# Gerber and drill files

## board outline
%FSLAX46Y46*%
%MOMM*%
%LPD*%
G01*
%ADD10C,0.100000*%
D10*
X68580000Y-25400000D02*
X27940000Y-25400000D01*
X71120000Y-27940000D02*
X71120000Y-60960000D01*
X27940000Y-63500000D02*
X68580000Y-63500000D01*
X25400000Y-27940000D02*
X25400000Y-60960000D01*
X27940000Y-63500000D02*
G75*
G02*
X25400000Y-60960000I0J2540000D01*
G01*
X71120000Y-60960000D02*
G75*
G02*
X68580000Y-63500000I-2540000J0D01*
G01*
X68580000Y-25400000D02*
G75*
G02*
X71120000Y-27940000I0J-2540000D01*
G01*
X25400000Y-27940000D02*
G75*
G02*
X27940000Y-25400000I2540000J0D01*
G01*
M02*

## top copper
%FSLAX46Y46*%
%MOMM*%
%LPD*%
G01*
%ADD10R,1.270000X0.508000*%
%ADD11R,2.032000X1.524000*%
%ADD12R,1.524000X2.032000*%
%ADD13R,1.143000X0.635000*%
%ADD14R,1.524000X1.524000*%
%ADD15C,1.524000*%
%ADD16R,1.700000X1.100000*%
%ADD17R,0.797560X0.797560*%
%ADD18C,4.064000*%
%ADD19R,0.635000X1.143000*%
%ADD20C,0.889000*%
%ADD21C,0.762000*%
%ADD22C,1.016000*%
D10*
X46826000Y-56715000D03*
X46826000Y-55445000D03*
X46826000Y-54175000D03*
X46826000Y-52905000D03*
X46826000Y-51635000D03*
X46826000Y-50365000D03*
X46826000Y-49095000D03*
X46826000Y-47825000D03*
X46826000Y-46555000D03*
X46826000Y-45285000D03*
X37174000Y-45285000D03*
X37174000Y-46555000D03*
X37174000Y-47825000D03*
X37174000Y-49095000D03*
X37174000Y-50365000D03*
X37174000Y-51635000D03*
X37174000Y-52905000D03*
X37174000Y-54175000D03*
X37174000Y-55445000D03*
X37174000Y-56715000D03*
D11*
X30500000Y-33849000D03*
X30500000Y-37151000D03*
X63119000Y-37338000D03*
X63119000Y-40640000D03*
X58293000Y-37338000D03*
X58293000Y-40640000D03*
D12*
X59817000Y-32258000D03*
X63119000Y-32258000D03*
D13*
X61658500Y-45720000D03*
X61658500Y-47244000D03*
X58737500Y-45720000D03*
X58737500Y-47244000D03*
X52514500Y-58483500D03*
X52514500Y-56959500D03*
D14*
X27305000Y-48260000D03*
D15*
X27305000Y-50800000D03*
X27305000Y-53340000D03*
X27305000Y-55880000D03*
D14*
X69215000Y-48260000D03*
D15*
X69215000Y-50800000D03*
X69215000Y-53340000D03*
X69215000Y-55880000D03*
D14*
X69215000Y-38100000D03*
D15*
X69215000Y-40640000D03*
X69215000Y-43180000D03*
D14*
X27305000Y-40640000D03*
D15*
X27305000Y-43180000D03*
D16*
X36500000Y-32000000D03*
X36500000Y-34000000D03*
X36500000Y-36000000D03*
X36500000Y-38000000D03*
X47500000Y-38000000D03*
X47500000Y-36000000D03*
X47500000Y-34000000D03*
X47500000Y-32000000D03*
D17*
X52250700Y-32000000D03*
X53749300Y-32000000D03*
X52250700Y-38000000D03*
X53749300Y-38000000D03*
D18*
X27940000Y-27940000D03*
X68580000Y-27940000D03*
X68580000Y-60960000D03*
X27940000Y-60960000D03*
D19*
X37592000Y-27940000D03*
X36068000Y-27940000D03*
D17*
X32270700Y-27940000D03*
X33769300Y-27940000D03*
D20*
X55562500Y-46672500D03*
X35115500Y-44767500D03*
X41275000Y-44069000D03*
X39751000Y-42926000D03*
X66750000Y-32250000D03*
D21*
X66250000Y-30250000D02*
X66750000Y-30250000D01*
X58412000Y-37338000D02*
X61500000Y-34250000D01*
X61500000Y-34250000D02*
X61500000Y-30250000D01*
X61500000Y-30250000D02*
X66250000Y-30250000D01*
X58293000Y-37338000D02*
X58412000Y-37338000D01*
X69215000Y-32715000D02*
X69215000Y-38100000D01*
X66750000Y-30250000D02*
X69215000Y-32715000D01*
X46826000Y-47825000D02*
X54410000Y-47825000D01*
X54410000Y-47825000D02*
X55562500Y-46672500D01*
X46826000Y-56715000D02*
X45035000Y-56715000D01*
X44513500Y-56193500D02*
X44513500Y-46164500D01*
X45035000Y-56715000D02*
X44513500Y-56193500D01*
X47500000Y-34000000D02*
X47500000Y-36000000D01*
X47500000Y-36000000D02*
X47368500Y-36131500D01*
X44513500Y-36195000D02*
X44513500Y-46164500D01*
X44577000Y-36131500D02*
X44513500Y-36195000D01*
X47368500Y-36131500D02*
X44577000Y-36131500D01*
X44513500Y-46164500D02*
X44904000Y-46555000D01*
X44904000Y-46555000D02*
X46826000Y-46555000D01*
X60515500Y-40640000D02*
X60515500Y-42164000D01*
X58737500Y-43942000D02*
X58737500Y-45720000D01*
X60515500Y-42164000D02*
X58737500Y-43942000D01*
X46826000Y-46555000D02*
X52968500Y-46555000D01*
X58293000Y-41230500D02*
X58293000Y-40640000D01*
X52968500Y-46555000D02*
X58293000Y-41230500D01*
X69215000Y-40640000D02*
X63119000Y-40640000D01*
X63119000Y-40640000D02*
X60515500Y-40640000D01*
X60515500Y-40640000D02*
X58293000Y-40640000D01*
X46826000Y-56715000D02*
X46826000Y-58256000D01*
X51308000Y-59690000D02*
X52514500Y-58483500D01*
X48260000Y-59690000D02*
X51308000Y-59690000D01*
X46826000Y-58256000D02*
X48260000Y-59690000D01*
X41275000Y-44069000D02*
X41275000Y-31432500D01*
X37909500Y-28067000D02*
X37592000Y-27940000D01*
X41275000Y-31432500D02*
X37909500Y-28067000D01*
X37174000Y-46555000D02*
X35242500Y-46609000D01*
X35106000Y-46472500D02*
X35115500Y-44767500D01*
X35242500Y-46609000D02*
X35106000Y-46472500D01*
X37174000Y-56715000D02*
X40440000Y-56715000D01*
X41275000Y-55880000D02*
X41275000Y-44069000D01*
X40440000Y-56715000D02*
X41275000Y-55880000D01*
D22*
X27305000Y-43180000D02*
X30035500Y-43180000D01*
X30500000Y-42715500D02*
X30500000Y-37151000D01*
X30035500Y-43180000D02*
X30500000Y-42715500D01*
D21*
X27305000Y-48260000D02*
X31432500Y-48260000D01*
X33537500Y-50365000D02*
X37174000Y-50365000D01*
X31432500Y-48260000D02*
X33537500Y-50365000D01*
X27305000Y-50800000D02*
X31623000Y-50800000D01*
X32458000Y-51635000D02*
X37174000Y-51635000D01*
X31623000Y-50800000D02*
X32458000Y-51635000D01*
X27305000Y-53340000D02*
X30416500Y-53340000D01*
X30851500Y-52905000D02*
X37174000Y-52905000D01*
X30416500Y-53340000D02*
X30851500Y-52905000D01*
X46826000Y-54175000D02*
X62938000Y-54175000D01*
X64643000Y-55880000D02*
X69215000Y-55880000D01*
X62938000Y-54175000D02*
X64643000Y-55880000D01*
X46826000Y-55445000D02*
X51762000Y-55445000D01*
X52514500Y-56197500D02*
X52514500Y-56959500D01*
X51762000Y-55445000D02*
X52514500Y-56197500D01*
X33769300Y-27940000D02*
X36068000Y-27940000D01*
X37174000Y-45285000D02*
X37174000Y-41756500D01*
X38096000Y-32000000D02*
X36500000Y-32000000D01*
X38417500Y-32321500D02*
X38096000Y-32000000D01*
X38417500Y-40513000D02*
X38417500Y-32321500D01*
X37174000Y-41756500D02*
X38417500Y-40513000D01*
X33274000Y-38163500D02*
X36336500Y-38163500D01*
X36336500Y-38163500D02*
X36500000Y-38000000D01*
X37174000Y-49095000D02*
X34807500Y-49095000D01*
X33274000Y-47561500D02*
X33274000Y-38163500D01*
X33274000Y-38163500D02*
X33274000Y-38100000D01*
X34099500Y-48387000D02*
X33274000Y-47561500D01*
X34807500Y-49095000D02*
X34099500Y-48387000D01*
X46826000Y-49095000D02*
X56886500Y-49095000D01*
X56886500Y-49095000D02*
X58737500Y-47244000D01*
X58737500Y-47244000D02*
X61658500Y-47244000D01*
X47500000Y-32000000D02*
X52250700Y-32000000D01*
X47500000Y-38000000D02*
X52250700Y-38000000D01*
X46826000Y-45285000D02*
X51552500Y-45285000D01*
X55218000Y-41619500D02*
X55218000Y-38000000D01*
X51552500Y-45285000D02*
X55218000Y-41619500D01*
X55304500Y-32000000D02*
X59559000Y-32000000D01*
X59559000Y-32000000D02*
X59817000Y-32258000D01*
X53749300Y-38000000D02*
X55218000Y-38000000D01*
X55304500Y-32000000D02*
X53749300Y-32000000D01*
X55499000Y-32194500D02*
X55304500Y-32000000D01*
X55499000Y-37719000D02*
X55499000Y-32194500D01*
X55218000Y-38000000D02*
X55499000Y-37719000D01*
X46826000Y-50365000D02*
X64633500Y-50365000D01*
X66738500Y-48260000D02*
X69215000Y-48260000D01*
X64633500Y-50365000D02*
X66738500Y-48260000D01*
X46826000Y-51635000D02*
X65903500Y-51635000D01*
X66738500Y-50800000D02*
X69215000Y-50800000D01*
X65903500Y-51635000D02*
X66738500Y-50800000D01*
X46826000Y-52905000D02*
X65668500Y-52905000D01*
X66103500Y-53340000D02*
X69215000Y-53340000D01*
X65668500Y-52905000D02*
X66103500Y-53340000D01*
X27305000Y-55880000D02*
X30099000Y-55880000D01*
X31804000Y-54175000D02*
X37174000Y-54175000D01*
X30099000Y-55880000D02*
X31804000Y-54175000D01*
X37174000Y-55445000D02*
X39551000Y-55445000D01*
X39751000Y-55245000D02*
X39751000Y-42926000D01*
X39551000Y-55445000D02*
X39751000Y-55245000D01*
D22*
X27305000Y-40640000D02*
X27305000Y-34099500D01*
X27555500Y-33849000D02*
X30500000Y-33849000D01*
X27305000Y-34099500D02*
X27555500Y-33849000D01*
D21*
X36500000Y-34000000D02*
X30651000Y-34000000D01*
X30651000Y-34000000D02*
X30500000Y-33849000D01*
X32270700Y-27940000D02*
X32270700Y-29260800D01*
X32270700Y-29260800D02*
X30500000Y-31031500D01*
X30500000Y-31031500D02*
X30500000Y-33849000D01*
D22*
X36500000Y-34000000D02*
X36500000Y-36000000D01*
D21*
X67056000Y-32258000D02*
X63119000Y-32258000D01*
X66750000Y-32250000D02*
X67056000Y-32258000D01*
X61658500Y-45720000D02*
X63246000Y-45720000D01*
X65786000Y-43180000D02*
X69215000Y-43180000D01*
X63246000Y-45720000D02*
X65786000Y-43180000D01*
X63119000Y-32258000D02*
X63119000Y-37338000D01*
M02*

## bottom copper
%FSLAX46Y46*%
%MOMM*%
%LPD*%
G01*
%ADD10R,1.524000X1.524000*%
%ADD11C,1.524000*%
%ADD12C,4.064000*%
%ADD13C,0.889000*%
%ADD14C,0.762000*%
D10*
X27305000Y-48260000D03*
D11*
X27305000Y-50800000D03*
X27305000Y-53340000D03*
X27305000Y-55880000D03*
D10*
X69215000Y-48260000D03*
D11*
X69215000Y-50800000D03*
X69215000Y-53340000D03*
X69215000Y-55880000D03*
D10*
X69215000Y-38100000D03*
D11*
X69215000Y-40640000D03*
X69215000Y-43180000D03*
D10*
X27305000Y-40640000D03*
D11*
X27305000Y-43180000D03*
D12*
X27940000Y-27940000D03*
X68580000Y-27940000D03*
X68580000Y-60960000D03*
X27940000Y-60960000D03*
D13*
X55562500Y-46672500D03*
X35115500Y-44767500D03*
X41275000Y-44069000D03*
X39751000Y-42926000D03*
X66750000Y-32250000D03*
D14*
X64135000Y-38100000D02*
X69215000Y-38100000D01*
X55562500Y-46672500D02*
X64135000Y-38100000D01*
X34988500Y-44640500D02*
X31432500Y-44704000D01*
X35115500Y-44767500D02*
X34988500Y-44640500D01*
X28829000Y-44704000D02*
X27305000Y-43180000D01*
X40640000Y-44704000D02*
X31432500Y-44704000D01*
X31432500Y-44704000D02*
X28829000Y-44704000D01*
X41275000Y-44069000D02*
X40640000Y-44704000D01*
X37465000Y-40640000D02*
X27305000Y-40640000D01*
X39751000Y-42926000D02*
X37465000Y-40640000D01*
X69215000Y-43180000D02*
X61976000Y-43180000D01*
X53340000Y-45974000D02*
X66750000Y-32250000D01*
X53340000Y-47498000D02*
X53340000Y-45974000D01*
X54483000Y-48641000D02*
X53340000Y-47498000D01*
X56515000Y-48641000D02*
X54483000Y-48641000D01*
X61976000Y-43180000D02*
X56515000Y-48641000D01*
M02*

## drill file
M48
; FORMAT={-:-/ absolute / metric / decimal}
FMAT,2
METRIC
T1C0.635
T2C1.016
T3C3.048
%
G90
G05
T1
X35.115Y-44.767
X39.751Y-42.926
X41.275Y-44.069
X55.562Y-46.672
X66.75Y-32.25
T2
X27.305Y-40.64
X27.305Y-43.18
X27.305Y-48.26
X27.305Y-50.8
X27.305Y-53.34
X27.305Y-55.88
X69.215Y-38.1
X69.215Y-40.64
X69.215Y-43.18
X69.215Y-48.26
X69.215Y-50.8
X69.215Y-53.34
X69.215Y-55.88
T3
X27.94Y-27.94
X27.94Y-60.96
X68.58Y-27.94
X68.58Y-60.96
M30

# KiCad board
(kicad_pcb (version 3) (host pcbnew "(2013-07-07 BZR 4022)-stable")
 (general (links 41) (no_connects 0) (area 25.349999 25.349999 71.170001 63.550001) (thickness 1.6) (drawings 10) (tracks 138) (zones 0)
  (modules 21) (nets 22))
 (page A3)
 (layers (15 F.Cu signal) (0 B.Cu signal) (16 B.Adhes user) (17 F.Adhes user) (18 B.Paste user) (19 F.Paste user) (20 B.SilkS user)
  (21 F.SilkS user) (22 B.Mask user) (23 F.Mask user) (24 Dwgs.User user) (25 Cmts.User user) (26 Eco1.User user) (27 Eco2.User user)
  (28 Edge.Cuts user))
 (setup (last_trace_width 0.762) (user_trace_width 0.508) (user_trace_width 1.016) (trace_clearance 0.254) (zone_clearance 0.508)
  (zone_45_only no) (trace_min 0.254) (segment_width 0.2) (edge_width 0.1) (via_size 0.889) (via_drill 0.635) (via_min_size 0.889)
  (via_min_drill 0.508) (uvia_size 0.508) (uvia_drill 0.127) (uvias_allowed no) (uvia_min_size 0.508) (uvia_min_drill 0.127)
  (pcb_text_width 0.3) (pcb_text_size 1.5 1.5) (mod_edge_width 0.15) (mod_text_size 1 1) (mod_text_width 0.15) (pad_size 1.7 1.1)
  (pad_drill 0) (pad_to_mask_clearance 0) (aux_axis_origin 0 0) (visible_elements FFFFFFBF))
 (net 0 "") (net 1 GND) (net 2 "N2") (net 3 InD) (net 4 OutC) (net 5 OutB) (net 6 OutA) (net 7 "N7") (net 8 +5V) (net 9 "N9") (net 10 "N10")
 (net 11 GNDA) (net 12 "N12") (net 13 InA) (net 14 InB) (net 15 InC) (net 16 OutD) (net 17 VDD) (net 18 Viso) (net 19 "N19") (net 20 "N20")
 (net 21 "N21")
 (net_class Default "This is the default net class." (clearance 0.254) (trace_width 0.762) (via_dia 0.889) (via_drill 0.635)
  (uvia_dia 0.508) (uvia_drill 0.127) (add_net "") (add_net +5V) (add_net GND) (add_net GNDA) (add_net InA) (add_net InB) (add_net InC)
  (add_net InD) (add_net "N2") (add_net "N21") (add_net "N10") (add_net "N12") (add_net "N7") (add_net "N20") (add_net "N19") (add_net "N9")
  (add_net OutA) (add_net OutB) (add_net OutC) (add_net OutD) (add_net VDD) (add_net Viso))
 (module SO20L (layer F.Cu) (at 42 51 270)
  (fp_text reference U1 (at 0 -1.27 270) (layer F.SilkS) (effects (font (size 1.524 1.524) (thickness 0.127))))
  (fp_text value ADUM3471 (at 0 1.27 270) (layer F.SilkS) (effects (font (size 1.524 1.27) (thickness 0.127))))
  (pad 11 smd rect (at 5.715 -4.826 270) (size 0.508 1.27) (layers F.Cu F.Paste F.Mask) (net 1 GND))
  (pad 12 smd rect (at 4.445 -4.826 270) (size 0.508 1.27) (layers F.Cu F.Paste F.Mask) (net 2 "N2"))
  (pad 13 smd rect (at 3.175 -4.826 270) (size 0.508 1.27) (layers F.Cu F.Paste F.Mask) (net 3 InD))
  (pad 14 smd rect (at 1.905 -4.826 270) (size 0.508 1.27) (layers F.Cu F.Paste F.Mask) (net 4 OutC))
  (pad 15 smd rect (at 0.635 -4.826 270) (size 0.508 1.27) (layers F.Cu F.Paste F.Mask) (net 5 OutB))
  (pad 16 smd rect (at -0.635 -4.826 270) (size 0.508 1.27) (layers F.Cu F.Paste F.Mask) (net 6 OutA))
  (pad 17 smd rect (at -1.905 -4.826 270) (size 0.508 1.27) (layers F.Cu F.Paste F.Mask) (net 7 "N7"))
  (pad 18 smd rect (at -3.175 -4.826 270) (size 0.508 1.27) (layers F.Cu F.Paste F.Mask) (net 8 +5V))
  (pad 19 smd rect (at -4.445 -4.826 270) (size 0.508 1.27) (layers F.Cu F.Paste F.Mask) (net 1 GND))
  (pad 20 smd rect (at -5.715 -4.826 270) (size 0.508 1.27) (layers F.Cu F.Paste F.Mask) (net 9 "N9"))
  (pad 1 smd rect (at -5.715 4.826 270) (size 0.508 1.27) (layers F.Cu F.Paste F.Mask) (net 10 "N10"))
  (pad 2 smd rect (at -4.445 4.826 270) (size 0.508 1.27) (layers F.Cu F.Paste F.Mask) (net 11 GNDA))
  (pad 3 smd rect (at -3.175 4.826 270) (size 0.508 1.27) (layers F.Cu F.Paste F.Mask))
  (pad 4 smd rect (at -1.905 4.826 270) (size 0.508 1.27) (layers F.Cu F.Paste F.Mask) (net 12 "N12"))
  (pad 5 smd rect (at -0.635 4.826 270) (size 0.508 1.27) (layers F.Cu F.Paste F.Mask) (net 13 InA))
  (pad 6 smd rect (at 0.635 4.826 270) (size 0.508 1.27) (layers F.Cu F.Paste F.Mask) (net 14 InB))
  (pad 7 smd rect (at 1.905 4.826 270) (size 0.508 1.27) (layers F.Cu F.Paste F.Mask) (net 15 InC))
  (pad 8 smd rect (at 3.175 4.826 270) (size 0.508 1.27) (layers F.Cu F.Paste F.Mask) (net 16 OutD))
  (pad 9 smd rect (at 4.445 4.826 270) (size 0.508 1.27) (layers F.Cu F.Paste F.Mask) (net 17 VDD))
  (pad 10 smd rect (at 5.715 4.826 270) (size 0.508 1.27) (layers F.Cu F.Paste F.Mask) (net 11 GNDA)))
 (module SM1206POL (layer F.Cu) (at 30.5 35.5 270)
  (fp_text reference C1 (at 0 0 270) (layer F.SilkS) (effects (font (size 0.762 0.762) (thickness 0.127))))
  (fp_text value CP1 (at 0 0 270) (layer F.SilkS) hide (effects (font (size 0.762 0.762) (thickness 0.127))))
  (pad 1 smd rect (at -1.651 0 270) (size 1.524 2.032) (layers F.Cu F.Paste F.Mask) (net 17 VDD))
  (pad 2 smd rect (at 1.651 0 270) (size 1.524 2.032) (layers F.Cu F.Paste F.Mask) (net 11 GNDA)))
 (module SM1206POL (layer F.Cu) (at 63.119 38.989 270)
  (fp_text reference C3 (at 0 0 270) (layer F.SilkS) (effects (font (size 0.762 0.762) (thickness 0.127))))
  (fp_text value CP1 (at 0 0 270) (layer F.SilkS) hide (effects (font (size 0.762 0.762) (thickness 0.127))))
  (pad 1 smd rect (at -1.651 0 270) (size 1.524 2.032) (layers F.Cu F.Paste F.Mask) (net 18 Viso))
  (pad 2 smd rect (at 1.651 0 270) (size 1.524 2.032) (layers F.Cu F.Paste F.Mask) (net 1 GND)))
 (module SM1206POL (layer F.Cu) (at 58.293 38.989 270)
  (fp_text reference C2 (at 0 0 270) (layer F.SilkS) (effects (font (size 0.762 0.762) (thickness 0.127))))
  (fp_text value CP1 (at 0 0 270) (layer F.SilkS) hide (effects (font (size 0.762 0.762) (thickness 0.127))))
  (pad 1 smd rect (at -1.651 0 270) (size 1.524 2.032) (layers F.Cu F.Paste F.Mask) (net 8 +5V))
  (pad 2 smd rect (at 1.651 0 270) (size 1.524 2.032) (layers F.Cu F.Paste F.Mask) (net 1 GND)))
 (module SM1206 (layer F.Cu) (at 61.468 32.258)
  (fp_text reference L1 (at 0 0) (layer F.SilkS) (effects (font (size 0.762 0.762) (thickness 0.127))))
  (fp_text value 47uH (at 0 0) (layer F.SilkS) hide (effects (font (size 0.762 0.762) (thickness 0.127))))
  (pad 1 smd rect (at -1.651 0) (size 1.524 2.032) (layers F.Cu F.Paste F.Mask) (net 9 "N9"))
  (pad 2 smd rect (at 1.651 0) (size 1.524 2.032) (layers F.Cu F.Paste F.Mask) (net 18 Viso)))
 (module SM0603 (layer F.Cu) (at 61.6585 46.482 270)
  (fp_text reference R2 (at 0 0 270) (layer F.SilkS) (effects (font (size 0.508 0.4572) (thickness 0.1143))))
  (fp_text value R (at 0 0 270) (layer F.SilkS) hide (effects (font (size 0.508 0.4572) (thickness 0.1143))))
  (pad 1 smd rect (at -0.762 0 270) (size 0.635 1.143) (layers F.Cu F.Paste F.Mask) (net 18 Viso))
  (pad 2 smd rect (at 0.762 0 270) (size 0.635 1.143) (layers F.Cu F.Paste F.Mask) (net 7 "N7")))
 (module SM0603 (layer F.Cu) (at 58.7375 46.482 270)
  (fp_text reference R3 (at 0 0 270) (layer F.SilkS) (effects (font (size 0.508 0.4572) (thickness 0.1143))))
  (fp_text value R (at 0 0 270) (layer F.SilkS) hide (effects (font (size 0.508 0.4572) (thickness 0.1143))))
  (pad 1 smd rect (at -0.762 0 270) (size 0.635 1.143) (layers F.Cu F.Paste F.Mask) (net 1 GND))
  (pad 2 smd rect (at 0.762 0 270) (size 0.635 1.143) (layers F.Cu F.Paste F.Mask) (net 7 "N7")))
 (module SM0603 (layer F.Cu) (at 52.5145 57.7215 90)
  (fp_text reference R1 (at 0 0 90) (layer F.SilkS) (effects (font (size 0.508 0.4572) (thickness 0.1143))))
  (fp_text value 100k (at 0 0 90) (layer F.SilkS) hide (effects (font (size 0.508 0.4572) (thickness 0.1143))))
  (pad 1 smd rect (at -0.762 0 90) (size 0.635 1.143) (layers F.Cu F.Paste F.Mask) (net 1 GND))
  (pad 2 smd rect (at 0.762 0 90) (size 0.635 1.143) (layers F.Cu F.Paste F.Mask) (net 2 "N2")))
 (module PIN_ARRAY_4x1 (layer F.Cu) (at 27.305 52.07 270)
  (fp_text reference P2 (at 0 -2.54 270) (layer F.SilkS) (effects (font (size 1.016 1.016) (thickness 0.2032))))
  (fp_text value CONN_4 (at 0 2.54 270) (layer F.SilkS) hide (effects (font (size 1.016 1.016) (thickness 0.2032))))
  (pad 1 thru_hole rect (at -3.81 0 270) (size 1.524 1.524) (drill 1.016) (layers *.Cu *.Mask F.SilkS) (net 13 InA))
  (pad 2 thru_hole circle (at -1.27 0 270) (size 1.524 1.524) (drill 1.016) (layers *.Cu *.Mask F.SilkS) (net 14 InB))
  (pad 3 thru_hole circle (at 1.27 0 270) (size 1.524 1.524) (drill 1.016) (layers *.Cu *.Mask F.SilkS) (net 15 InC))
  (pad 4 thru_hole circle (at 3.81 0 270) (size 1.524 1.524) (drill 1.016) (layers *.Cu *.Mask F.SilkS) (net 16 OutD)))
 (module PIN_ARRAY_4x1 (layer F.Cu) (at 69.215 52.07 270)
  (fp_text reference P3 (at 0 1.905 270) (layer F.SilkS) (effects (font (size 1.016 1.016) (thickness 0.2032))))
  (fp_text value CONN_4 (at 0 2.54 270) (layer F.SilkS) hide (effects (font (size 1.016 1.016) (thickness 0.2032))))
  (pad 1 thru_hole rect (at -3.81 0 270) (size 1.524 1.524) (drill 1.016) (layers *.Cu *.Mask F.SilkS) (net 6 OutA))
  (pad 2 thru_hole circle (at -1.27 0 270) (size 1.524 1.524) (drill 1.016) (layers *.Cu *.Mask F.SilkS) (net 5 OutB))
  (pad 3 thru_hole circle (at 1.27 0 270) (size 1.524 1.524) (drill 1.016) (layers *.Cu *.Mask F.SilkS) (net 4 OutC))
  (pad 4 thru_hole circle (at 3.81 0 270) (size 1.524 1.524) (drill 1.016) (layers *.Cu *.Mask F.SilkS) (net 3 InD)))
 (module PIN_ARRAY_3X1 (layer F.Cu) (at 69.215 40.64 270)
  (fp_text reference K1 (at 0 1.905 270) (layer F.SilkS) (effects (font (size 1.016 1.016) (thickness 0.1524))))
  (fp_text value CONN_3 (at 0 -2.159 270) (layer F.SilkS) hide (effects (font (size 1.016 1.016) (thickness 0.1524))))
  (pad 1 thru_hole rect (at -2.54 0 270) (size 1.524 1.524) (drill 1.016) (layers *.Cu *.Mask F.SilkS) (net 8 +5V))
  (pad 2 thru_hole circle (at 0 0 270) (size 1.524 1.524) (drill 1.016) (layers *.Cu *.Mask F.SilkS) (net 1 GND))
  (pad 3 thru_hole circle (at 2.54 0 270) (size 1.524 1.524) (drill 1.016) (layers *.Cu *.Mask F.SilkS) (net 18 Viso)))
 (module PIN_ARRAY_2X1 (layer F.Cu) (at 27.305 41.91 270)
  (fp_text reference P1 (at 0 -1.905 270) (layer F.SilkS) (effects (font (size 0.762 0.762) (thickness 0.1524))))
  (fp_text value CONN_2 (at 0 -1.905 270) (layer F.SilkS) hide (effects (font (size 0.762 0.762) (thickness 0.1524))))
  (pad 1 thru_hole rect (at -1.27 0 270) (size 1.524 1.524) (drill 1.016) (layers *.Cu *.Mask F.SilkS) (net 17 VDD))
  (pad 2 thru_hole circle (at 1.27 0 270) (size 1.524 1.524) (drill 1.016) (layers *.Cu *.Mask F.SilkS) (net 11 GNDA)))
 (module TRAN (layer F.Cu) (at 42 35)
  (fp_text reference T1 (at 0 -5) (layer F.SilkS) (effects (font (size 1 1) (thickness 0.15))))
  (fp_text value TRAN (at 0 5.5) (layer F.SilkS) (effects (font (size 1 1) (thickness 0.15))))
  (pad 1 smd rect (at -5.5 -3) (size 1.7 1.1) (layers F.Cu F.Paste F.Mask) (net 10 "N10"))
  (pad 2 smd rect (at -5.5 -1) (size 1.7 1.1) (layers F.Cu F.Paste F.Mask) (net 17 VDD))
  (pad 3 smd rect (at -5.5 1) (size 1.7 1.1) (layers F.Cu F.Paste F.Mask) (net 17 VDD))
  (pad 4 smd rect (at -5.5 3) (size 1.7 1.1) (layers F.Cu F.Paste F.Mask) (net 12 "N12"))
  (pad 5 smd rect (at 5.5 3) (size 1.7 1.1) (layers F.Cu F.Paste F.Mask) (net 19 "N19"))
  (pad 6 smd rect (at 5.5 1) (size 1.7 1.1) (layers F.Cu F.Paste F.Mask) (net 1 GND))
  (pad 7 smd rect (at 5.5 -1) (size 1.7 1.1) (layers F.Cu F.Paste F.Mask) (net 1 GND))
  (pad 8 smd rect (at 5.5 -3) (size 1.7 1.1) (layers F.Cu F.Paste F.Mask) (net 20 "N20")))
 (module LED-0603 (layer F.Cu) (at 53 32)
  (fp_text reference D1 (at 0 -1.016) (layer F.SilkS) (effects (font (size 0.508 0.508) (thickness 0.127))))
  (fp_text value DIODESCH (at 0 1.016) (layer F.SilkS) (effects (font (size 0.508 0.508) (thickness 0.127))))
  (pad 1 smd rect (at -0.7493 0) (size 0.79756 0.79756) (layers F.Cu F.Paste F.Mask) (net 20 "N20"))
  (pad 2 smd rect (at 0.7493 0) (size 0.79756 0.79756) (layers F.Cu F.Paste F.Mask) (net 9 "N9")))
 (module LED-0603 (layer F.Cu) (at 53 38)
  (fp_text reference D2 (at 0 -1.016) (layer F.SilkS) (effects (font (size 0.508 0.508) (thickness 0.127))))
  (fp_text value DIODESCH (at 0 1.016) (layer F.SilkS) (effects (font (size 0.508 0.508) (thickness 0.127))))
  (pad 1 smd rect (at -0.7493 0) (size 0.79756 0.79756) (layers F.Cu F.Paste F.Mask) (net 19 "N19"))
  (pad 2 smd rect (at 0.7493 0) (size 0.79756 0.79756) (layers F.Cu F.Paste F.Mask) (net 9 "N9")))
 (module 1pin (layer F.Cu) (at 27.94 27.94)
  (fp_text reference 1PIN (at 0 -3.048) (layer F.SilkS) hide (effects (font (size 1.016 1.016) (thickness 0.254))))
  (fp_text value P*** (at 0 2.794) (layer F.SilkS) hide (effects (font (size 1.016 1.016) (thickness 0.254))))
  (pad 1 thru_hole circle (at 0 0) (size 4.064 4.064) (drill 3.048) (layers *.Cu *.Mask F.SilkS)))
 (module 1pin (layer F.Cu) (at 68.58 27.94)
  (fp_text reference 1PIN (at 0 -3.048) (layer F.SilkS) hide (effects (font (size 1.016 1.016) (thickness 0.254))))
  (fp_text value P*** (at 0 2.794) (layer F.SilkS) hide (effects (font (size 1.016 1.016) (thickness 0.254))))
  (pad 1 thru_hole circle (at 0 0) (size 4.064 4.064) (drill 3.048) (layers *.Cu *.Mask F.SilkS)))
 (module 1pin (layer F.Cu) (at 68.58 60.96)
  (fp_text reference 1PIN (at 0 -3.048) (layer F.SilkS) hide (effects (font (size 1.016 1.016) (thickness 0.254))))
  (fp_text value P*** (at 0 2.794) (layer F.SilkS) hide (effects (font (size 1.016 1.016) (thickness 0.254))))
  (pad 1 thru_hole circle (at 0 0) (size 4.064 4.064) (drill 3.048) (layers *.Cu *.Mask F.SilkS)))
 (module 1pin (layer F.Cu) (at 27.94 60.96)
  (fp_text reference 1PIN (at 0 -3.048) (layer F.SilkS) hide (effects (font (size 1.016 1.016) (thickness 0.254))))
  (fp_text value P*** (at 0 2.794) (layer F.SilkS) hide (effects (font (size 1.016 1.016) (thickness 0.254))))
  (pad 1 thru_hole circle (at 0 0) (size 4.064 4.064) (drill 3.048) (layers *.Cu *.Mask F.SilkS)))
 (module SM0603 (layer F.Cu) (at 36.83 27.94 180)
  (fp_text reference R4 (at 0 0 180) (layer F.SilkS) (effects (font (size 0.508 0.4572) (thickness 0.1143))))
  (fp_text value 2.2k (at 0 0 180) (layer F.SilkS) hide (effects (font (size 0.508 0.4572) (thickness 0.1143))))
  (pad 1 smd rect (at -0.762 0 180) (size 0.635 1.143) (layers F.Cu F.Paste F.Mask) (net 11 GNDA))
  (pad 2 smd rect (at 0.762 0 180) (size 0.635 1.143) (layers F.Cu F.Paste F.Mask) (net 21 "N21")))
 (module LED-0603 (layer F.Cu) (at 33.02 27.94)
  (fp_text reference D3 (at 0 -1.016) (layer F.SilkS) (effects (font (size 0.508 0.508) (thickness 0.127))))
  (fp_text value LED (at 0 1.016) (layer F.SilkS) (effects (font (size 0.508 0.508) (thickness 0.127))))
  (pad 1 smd rect (at -0.7493 0) (size 0.79756 0.79756) (layers F.Cu F.Paste F.Mask) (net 17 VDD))
  (pad 2 smd rect (at 0.7493 0) (size 0.79756 0.79756) (layers F.Cu F.Paste F.Mask) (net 21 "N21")))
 (gr_line (start 68.58 25.4) (end 27.94 25.4) (angle 90) (layer Edge.Cuts) (width 0.1))
 (gr_line (start 71.12 27.94) (end 71.12 60.96) (angle 90) (layer Edge.Cuts) (width 0.1))
 (gr_line (start 27.94 63.5) (end 68.58 63.5) (angle 90) (layer Edge.Cuts) (width 0.1))
 (gr_line (start 25.4 27.94) (end 25.4 60.96) (angle 90) (layer Edge.Cuts) (width 0.1))
 (gr_arc (start 27.94 60.96) (end 27.94 63.5) (angle 90) (layer Edge.Cuts) (width 0.1))
 (gr_arc (start 68.58 60.96) (end 71.12 60.96) (angle 90) (layer Edge.Cuts) (width 0.1))
 (gr_arc (start 68.58 27.94) (end 68.58 25.4) (angle 90) (layer Edge.Cuts) (width 0.1))
 (gr_arc (start 27.94 27.94) (end 25.4 27.94) (angle 90) (layer Edge.Cuts) (width 0.1))
 (segment (start 66.25 30.25) (end 66.75 30.25) (width 0.762) (layer F.Cu) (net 8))
 (segment (start 58.412 37.338) (end 61.5 34.25) (width 0.762) (layer F.Cu) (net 8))
 (segment (start 61.5 34.25) (end 61.5 30.25) (width 0.762) (layer F.Cu) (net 8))
 (segment (start 61.5 30.25) (end 66.25 30.25) (width 0.762) (layer F.Cu) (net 8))
 (segment (start 58.293 37.338) (end 58.412 37.338) (width 0.762) (layer F.Cu) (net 8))
 (segment (start 69.215 32.715) (end 69.215 38.1) (width 0.762) (layer F.Cu) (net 8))
 (segment (start 66.75 30.25) (end 69.215 32.715) (width 0.762) (layer F.Cu) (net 8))
 (segment (start 46.826 47.825) (end 54.41 47.825) (width 0.762) (layer F.Cu) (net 8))
 (segment (start 64.135 38.1) (end 69.215 38.1) (width 0.762) (layer B.Cu) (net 8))
 (segment (start 55.5625 46.6725) (end 64.135 38.1) (width 0.762) (layer B.Cu) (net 8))
 (via (at 55.5625 46.6725) (size 0.889) (layers F.Cu B.Cu) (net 8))
 (segment (start 54.41 47.825) (end 55.5625 46.6725) (width 0.762) (layer F.Cu) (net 8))
 (segment (start 46.826 56.715) (end 45.035 56.715) (width 0.762) (layer F.Cu) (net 1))
 (segment (start 44.5135 56.1935) (end 44.5135 46.1645) (width 0.762) (layer F.Cu) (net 1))
 (segment (start 45.035 56.715) (end 44.5135 56.1935) (width 0.762) (layer F.Cu) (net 1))
 (segment (start 47.5 34) (end 47.5 36) (width 0.762) (layer F.Cu) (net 1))
 (segment (start 47.5 36) (end 47.3685 36.1315) (width 0.762) (layer F.Cu) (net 1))
 (segment (start 44.5135 36.195) (end 44.5135 46.1645) (width 0.762) (layer F.Cu) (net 1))
 (segment (start 44.577 36.1315) (end 44.5135 36.195) (width 0.762) (layer F.Cu) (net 1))
 (segment (start 47.3685 36.1315) (end 44.577 36.1315) (width 0.762) (layer F.Cu) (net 1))
 (segment (start 44.5135 46.1645) (end 44.904 46.555) (width 0.762) (layer F.Cu) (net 1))
 (segment (start 44.904 46.555) (end 46.826 46.555) (width 0.762) (layer F.Cu) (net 1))
 (segment (start 60.5155 40.64) (end 60.5155 42.164) (width 0.762) (layer F.Cu) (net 1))
 (segment (start 58.7375 43.942) (end 58.7375 45.72) (width 0.762) (layer F.Cu) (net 1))
 (segment (start 60.5155 42.164) (end 58.7375 43.942) (width 0.762) (layer F.Cu) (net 1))
 (segment (start 46.826 46.555) (end 52.9685 46.555) (width 0.762) (layer F.Cu) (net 1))
 (segment (start 58.293 41.2305) (end 58.293 40.64) (width 0.762) (layer F.Cu) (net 1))
 (segment (start 52.9685 46.555) (end 58.293 41.2305) (width 0.762) (layer F.Cu) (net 1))
 (segment (start 69.215 40.64) (end 63.119 40.64) (width 0.762) (layer F.Cu) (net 1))
 (segment (start 63.119 40.64) (end 60.5155 40.64) (width 0.762) (layer F.Cu) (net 1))
 (segment (start 60.5155 40.64) (end 58.293 40.64) (width 0.762) (layer F.Cu) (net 1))
 (segment (start 46.826 56.715) (end 46.826 58.256) (width 0.762) (layer F.Cu) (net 1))
 (segment (start 51.308 59.69) (end 52.5145 58.4835) (width 0.762) (layer F.Cu) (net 1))
 (segment (start 48.26 59.69) (end 51.308 59.69) (width 0.762) (layer F.Cu) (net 1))
 (segment (start 46.826 58.256) (end 48.26 59.69) (width 0.762) (layer F.Cu) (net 1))
 (segment (start 41.275 44.069) (end 41.275 31.4325) (width 0.762) (layer F.Cu) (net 11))
 (segment (start 37.9095 28.067) (end 37.592 27.94) (width 0.762) (layer F.Cu) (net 11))
 (segment (start 41.275 31.4325) (end 37.9095 28.067) (width 0.762) (layer F.Cu) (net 11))
 (segment (start 37.174 46.555) (end 35.2425 46.609) (width 0.762) (layer F.Cu) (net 11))
 (segment (start 34.9885 44.6405) (end 31.4325 44.704) (width 0.762) (layer B.Cu) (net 11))
 (segment (start 35.1155 44.7675) (end 34.9885 44.6405) (width 0.762) (layer B.Cu) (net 11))
 (via (at 35.1155 44.7675) (size 0.889) (layers F.Cu B.Cu) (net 11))
 (segment (start 35.106 46.4725) (end 35.1155 44.7675) (width 0.762) (layer F.Cu) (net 11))
 (segment (start 35.2425 46.609) (end 35.106 46.4725) (width 0.762) (layer F.Cu) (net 11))
 (segment (start 37.174 56.715) (end 40.44 56.715) (width 0.762) (layer F.Cu) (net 11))
 (segment (start 28.829 44.704) (end 27.305 43.18) (width 0.762) (layer B.Cu) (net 11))
 (segment (start 40.64 44.704) (end 31.4325 44.704) (width 0.762) (layer B.Cu) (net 11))
 (segment (start 31.4325 44.704) (end 28.829 44.704) (width 0.762) (layer B.Cu) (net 11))
 (segment (start 41.275 44.069) (end 40.64 44.704) (width 0.762) (layer B.Cu) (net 11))
 (via (at 41.275 44.069) (size 0.889) (layers F.Cu B.Cu) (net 11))
 (segment (start 41.275 55.88) (end 41.275 44.069) (width 0.762) (layer F.Cu) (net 11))
 (segment (start 40.44 56.715) (end 41.275 55.88) (width 0.762) (layer F.Cu) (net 11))
 (segment (start 27.305 43.18) (end 30.0355 43.18) (width 1.016) (layer F.Cu) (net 11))
 (segment (start 30.5 42.7155) (end 30.5 37.151) (width 1.016) (layer F.Cu) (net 11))
 (segment (start 30.0355 43.18) (end 30.5 42.7155) (width 1.016) (layer F.Cu) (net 11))
 (segment (start 27.305 48.26) (end 31.4325 48.26) (width 0.762) (layer F.Cu) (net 13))
 (segment (start 33.5375 50.365) (end 37.174 50.365) (width 0.762) (layer F.Cu) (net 13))
 (segment (start 31.4325 48.26) (end 33.5375 50.365) (width 0.762) (layer F.Cu) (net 13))
 (segment (start 27.305 50.8) (end 31.623 50.8) (width 0.762) (layer F.Cu) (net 14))
 (segment (start 32.458 51.635) (end 37.174 51.635) (width 0.762) (layer F.Cu) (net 14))
 (segment (start 31.623 50.8) (end 32.458 51.635) (width 0.762) (layer F.Cu) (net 14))
 (segment (start 27.305 53.34) (end 30.4165 53.34) (width 0.762) (layer F.Cu) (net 15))
 (segment (start 30.8515 52.905) (end 37.174 52.905) (width 0.762) (layer F.Cu) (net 15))
 (segment (start 30.4165 53.34) (end 30.8515 52.905) (width 0.762) (layer F.Cu) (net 15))
 (segment (start 46.826 54.175) (end 62.938 54.175) (width 0.762) (layer F.Cu) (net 3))
 (segment (start 64.643 55.88) (end 69.215 55.88) (width 0.762) (layer F.Cu) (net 3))
 (segment (start 62.938 54.175) (end 64.643 55.88) (width 0.762) (layer F.Cu) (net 3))
 (segment (start 46.826 55.445) (end 51.762 55.445) (width 0.762) (layer F.Cu) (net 2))
 (segment (start 52.5145 56.1975) (end 52.5145 56.9595) (width 0.762) (layer F.Cu) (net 2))
 (segment (start 51.762 55.445) (end 52.5145 56.1975) (width 0.762) (layer F.Cu) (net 2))
 (segment (start 33.7693 27.94) (end 36.068 27.94) (width 0.762) (layer F.Cu) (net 21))
 (segment (start 37.174 45.285) (end 37.174 41.7565) (width 0.762) (layer F.Cu) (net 10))
 (segment (start 38.096 32) (end 36.5 32) (width 0.762) (layer F.Cu) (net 10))
 (segment (start 38.4175 32.3215) (end 38.096 32) (width 0.762) (layer F.Cu) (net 10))
 (segment (start 38.4175 40.513) (end 38.4175 32.3215) (width 0.762) (layer F.Cu) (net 10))
 (segment (start 37.174 41.7565) (end 38.4175 40.513) (width 0.762) (layer F.Cu) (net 10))
 (segment (start 33.274 38.1635) (end 36.3365 38.1635) (width 0.762) (layer F.Cu) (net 12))
 (segment (start 36.3365 38.1635) (end 36.5 38) (width 0.762) (layer F.Cu) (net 12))
 (segment (start 37.174 49.095) (end 34.8075 49.095) (width 0.762) (layer F.Cu) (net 12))
 (segment (start 33.274 47.5615) (end 33.274 38.1635) (width 0.762) (layer F.Cu) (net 12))
 (segment (start 33.274 38.1635) (end 33.274 38.1) (width 0.762) (layer F.Cu) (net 12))
 (segment (start 34.0995 48.387) (end 33.274 47.5615) (width 0.762) (layer F.Cu) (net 12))
 (segment (start 34.8075 49.095) (end 34.0995 48.387) (width 0.762) (layer F.Cu) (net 12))
 (segment (start 46.826 49.095) (end 56.8865 49.095) (width 0.762) (layer F.Cu) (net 7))
 (segment (start 56.8865 49.095) (end 58.7375 47.244) (width 0.762) (layer F.Cu) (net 7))
 (segment (start 58.7375 47.244) (end 61.6585 47.244) (width 0.762) (layer F.Cu) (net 7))
 (segment (start 47.5 32) (end 52.2507 32) (width 0.762) (layer F.Cu) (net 20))
 (segment (start 47.5 38) (end 52.2507 38) (width 0.762) (layer F.Cu) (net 19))
 (segment (start 46.826 45.285) (end 51.5525 45.285) (width 0.762) (layer F.Cu) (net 9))
 (segment (start 55.218 41.6195) (end 55.218 38) (width 0.762) (layer F.Cu) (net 9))
 (segment (start 51.5525 45.285) (end 55.218 41.6195) (width 0.762) (layer F.Cu) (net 9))
 (segment (start 55.3045 32) (end 59.559 32) (width 0.762) (layer F.Cu) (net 9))
 (segment (start 59.559 32) (end 59.817 32.258) (width 0.762) (layer F.Cu) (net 9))
 (segment (start 53.7493 38) (end 55.218 38) (width 0.762) (layer F.Cu) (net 9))
 (segment (start 55.3045 32) (end 53.7493 32) (width 0.762) (layer F.Cu) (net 9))
 (segment (start 55.499 32.1945) (end 55.3045 32) (width 0.762) (layer F.Cu) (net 9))
 (segment (start 55.499 37.719) (end 55.499 32.1945) (width 0.762) (layer F.Cu) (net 9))
 (segment (start 55.218 38) (end 55.499 37.719) (width 0.762) (layer F.Cu) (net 9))
 (segment (start 46.826 50.365) (end 64.6335 50.365) (width 0.762) (layer F.Cu) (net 6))
 (segment (start 66.7385 48.26) (end 69.215 48.26) (width 0.762) (layer F.Cu) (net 6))
 (segment (start 64.6335 50.365) (end 66.7385 48.26) (width 0.762) (layer F.Cu) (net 6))
 (segment (start 46.826 51.635) (end 65.9035 51.635) (width 0.762) (layer F.Cu) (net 5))
 (segment (start 66.7385 50.8) (end 69.215 50.8) (width 0.762) (layer F.Cu) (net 5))
 (segment (start 65.9035 51.635) (end 66.7385 50.8) (width 0.762) (layer F.Cu) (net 5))
 (segment (start 46.826 52.905) (end 65.6685 52.905) (width 0.762) (layer F.Cu) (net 4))
 (segment (start 66.1035 53.34) (end 69.215 53.34) (width 0.762) (layer F.Cu) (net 4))
 (segment (start 65.6685 52.905) (end 66.1035 53.34) (width 0.762) (layer F.Cu) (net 4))
 (segment (start 27.305 55.88) (end 30.099 55.88) (width 0.762) (layer F.Cu) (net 16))
 (segment (start 31.804 54.175) (end 37.174 54.175) (width 0.762) (layer F.Cu) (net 16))
 (segment (start 30.099 55.88) (end 31.804 54.175) (width 0.762) (layer F.Cu) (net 16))
 (segment (start 37.174 55.445) (end 39.551 55.445) (width 0.762) (layer F.Cu) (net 17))
 (segment (start 37.465 40.64) (end 27.305 40.64) (width 0.762) (layer B.Cu) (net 17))
 (segment (start 39.751 42.926) (end 37.465 40.64) (width 0.762) (layer B.Cu) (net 17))
 (via (at 39.751 42.926) (size 0.889) (layers F.Cu B.Cu) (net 17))
 (segment (start 39.751 55.245) (end 39.751 42.926) (width 0.762) (layer F.Cu) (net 17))
 (segment (start 39.551 55.445) (end 39.751 55.245) (width 0.762) (layer F.Cu) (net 17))
 (segment (start 27.305 40.64) (end 27.305 34.0995) (width 1.016) (layer F.Cu) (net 17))
 (segment (start 27.5555 33.849) (end 30.5 33.849) (width 1.016) (layer F.Cu) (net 17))
 (segment (start 27.305 34.0995) (end 27.5555 33.849) (width 1.016) (layer F.Cu) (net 17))
 (segment (start 36.5 34) (end 30.651 34) (width 0.762) (layer F.Cu) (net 17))
 (segment (start 30.651 34) (end 30.5 33.849) (width 0.762) (layer F.Cu) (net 17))
 (segment (start 32.2707 27.94) (end 32.2707 29.2608) (width 0.762) (layer F.Cu) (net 17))
 (segment (start 32.2707 29.2608) (end 30.5 31.0315) (width 0.762) (layer F.Cu) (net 17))
 (segment (start 30.5 31.0315) (end 30.5 33.849) (width 0.762) (layer F.Cu) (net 17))
 (segment (start 36.5 34) (end 36.5 36) (width 1.016) (layer F.Cu) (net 17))
 (segment (start 69.215 43.18) (end 61.976 43.18) (width 0.762) (layer B.Cu) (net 18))
 (segment (start 67.056 32.258) (end 63.119 32.258) (width 0.762) (layer F.Cu) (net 18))
 (segment (start 66.75 32.25) (end 67.056 32.258) (width 0.762) (layer F.Cu) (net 18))
 (via (at 66.75 32.25) (size 0.889) (layers F.Cu B.Cu) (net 18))
 (segment (start 53.34 45.974) (end 66.75 32.25) (width 0.762) (layer B.Cu) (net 18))
 (segment (start 53.34 47.498) (end 53.34 45.974) (width 0.762) (layer B.Cu) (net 18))
 (segment (start 54.483 48.641) (end 53.34 47.498) (width 0.762) (layer B.Cu) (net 18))
 (segment (start 56.515 48.641) (end 54.483 48.641) (width 0.762) (layer B.Cu) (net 18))
 (segment (start 61.976 43.18) (end 56.515 48.641) (width 0.762) (layer B.Cu) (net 18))
 (segment (start 61.6585 45.72) (end 63.246 45.72) (width 0.762) (layer F.Cu) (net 18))
 (segment (start 65.786 43.18) (end 69.215 43.18) (width 0.762) (layer F.Cu) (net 18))
 (segment (start 63.246 45.72) (end 65.786 43.18) (width 0.762) (layer F.Cu) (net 18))
 (segment (start 63.119 32.258) (end 63.119 37.338) (width 0.762) (layer F.Cu) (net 18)))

